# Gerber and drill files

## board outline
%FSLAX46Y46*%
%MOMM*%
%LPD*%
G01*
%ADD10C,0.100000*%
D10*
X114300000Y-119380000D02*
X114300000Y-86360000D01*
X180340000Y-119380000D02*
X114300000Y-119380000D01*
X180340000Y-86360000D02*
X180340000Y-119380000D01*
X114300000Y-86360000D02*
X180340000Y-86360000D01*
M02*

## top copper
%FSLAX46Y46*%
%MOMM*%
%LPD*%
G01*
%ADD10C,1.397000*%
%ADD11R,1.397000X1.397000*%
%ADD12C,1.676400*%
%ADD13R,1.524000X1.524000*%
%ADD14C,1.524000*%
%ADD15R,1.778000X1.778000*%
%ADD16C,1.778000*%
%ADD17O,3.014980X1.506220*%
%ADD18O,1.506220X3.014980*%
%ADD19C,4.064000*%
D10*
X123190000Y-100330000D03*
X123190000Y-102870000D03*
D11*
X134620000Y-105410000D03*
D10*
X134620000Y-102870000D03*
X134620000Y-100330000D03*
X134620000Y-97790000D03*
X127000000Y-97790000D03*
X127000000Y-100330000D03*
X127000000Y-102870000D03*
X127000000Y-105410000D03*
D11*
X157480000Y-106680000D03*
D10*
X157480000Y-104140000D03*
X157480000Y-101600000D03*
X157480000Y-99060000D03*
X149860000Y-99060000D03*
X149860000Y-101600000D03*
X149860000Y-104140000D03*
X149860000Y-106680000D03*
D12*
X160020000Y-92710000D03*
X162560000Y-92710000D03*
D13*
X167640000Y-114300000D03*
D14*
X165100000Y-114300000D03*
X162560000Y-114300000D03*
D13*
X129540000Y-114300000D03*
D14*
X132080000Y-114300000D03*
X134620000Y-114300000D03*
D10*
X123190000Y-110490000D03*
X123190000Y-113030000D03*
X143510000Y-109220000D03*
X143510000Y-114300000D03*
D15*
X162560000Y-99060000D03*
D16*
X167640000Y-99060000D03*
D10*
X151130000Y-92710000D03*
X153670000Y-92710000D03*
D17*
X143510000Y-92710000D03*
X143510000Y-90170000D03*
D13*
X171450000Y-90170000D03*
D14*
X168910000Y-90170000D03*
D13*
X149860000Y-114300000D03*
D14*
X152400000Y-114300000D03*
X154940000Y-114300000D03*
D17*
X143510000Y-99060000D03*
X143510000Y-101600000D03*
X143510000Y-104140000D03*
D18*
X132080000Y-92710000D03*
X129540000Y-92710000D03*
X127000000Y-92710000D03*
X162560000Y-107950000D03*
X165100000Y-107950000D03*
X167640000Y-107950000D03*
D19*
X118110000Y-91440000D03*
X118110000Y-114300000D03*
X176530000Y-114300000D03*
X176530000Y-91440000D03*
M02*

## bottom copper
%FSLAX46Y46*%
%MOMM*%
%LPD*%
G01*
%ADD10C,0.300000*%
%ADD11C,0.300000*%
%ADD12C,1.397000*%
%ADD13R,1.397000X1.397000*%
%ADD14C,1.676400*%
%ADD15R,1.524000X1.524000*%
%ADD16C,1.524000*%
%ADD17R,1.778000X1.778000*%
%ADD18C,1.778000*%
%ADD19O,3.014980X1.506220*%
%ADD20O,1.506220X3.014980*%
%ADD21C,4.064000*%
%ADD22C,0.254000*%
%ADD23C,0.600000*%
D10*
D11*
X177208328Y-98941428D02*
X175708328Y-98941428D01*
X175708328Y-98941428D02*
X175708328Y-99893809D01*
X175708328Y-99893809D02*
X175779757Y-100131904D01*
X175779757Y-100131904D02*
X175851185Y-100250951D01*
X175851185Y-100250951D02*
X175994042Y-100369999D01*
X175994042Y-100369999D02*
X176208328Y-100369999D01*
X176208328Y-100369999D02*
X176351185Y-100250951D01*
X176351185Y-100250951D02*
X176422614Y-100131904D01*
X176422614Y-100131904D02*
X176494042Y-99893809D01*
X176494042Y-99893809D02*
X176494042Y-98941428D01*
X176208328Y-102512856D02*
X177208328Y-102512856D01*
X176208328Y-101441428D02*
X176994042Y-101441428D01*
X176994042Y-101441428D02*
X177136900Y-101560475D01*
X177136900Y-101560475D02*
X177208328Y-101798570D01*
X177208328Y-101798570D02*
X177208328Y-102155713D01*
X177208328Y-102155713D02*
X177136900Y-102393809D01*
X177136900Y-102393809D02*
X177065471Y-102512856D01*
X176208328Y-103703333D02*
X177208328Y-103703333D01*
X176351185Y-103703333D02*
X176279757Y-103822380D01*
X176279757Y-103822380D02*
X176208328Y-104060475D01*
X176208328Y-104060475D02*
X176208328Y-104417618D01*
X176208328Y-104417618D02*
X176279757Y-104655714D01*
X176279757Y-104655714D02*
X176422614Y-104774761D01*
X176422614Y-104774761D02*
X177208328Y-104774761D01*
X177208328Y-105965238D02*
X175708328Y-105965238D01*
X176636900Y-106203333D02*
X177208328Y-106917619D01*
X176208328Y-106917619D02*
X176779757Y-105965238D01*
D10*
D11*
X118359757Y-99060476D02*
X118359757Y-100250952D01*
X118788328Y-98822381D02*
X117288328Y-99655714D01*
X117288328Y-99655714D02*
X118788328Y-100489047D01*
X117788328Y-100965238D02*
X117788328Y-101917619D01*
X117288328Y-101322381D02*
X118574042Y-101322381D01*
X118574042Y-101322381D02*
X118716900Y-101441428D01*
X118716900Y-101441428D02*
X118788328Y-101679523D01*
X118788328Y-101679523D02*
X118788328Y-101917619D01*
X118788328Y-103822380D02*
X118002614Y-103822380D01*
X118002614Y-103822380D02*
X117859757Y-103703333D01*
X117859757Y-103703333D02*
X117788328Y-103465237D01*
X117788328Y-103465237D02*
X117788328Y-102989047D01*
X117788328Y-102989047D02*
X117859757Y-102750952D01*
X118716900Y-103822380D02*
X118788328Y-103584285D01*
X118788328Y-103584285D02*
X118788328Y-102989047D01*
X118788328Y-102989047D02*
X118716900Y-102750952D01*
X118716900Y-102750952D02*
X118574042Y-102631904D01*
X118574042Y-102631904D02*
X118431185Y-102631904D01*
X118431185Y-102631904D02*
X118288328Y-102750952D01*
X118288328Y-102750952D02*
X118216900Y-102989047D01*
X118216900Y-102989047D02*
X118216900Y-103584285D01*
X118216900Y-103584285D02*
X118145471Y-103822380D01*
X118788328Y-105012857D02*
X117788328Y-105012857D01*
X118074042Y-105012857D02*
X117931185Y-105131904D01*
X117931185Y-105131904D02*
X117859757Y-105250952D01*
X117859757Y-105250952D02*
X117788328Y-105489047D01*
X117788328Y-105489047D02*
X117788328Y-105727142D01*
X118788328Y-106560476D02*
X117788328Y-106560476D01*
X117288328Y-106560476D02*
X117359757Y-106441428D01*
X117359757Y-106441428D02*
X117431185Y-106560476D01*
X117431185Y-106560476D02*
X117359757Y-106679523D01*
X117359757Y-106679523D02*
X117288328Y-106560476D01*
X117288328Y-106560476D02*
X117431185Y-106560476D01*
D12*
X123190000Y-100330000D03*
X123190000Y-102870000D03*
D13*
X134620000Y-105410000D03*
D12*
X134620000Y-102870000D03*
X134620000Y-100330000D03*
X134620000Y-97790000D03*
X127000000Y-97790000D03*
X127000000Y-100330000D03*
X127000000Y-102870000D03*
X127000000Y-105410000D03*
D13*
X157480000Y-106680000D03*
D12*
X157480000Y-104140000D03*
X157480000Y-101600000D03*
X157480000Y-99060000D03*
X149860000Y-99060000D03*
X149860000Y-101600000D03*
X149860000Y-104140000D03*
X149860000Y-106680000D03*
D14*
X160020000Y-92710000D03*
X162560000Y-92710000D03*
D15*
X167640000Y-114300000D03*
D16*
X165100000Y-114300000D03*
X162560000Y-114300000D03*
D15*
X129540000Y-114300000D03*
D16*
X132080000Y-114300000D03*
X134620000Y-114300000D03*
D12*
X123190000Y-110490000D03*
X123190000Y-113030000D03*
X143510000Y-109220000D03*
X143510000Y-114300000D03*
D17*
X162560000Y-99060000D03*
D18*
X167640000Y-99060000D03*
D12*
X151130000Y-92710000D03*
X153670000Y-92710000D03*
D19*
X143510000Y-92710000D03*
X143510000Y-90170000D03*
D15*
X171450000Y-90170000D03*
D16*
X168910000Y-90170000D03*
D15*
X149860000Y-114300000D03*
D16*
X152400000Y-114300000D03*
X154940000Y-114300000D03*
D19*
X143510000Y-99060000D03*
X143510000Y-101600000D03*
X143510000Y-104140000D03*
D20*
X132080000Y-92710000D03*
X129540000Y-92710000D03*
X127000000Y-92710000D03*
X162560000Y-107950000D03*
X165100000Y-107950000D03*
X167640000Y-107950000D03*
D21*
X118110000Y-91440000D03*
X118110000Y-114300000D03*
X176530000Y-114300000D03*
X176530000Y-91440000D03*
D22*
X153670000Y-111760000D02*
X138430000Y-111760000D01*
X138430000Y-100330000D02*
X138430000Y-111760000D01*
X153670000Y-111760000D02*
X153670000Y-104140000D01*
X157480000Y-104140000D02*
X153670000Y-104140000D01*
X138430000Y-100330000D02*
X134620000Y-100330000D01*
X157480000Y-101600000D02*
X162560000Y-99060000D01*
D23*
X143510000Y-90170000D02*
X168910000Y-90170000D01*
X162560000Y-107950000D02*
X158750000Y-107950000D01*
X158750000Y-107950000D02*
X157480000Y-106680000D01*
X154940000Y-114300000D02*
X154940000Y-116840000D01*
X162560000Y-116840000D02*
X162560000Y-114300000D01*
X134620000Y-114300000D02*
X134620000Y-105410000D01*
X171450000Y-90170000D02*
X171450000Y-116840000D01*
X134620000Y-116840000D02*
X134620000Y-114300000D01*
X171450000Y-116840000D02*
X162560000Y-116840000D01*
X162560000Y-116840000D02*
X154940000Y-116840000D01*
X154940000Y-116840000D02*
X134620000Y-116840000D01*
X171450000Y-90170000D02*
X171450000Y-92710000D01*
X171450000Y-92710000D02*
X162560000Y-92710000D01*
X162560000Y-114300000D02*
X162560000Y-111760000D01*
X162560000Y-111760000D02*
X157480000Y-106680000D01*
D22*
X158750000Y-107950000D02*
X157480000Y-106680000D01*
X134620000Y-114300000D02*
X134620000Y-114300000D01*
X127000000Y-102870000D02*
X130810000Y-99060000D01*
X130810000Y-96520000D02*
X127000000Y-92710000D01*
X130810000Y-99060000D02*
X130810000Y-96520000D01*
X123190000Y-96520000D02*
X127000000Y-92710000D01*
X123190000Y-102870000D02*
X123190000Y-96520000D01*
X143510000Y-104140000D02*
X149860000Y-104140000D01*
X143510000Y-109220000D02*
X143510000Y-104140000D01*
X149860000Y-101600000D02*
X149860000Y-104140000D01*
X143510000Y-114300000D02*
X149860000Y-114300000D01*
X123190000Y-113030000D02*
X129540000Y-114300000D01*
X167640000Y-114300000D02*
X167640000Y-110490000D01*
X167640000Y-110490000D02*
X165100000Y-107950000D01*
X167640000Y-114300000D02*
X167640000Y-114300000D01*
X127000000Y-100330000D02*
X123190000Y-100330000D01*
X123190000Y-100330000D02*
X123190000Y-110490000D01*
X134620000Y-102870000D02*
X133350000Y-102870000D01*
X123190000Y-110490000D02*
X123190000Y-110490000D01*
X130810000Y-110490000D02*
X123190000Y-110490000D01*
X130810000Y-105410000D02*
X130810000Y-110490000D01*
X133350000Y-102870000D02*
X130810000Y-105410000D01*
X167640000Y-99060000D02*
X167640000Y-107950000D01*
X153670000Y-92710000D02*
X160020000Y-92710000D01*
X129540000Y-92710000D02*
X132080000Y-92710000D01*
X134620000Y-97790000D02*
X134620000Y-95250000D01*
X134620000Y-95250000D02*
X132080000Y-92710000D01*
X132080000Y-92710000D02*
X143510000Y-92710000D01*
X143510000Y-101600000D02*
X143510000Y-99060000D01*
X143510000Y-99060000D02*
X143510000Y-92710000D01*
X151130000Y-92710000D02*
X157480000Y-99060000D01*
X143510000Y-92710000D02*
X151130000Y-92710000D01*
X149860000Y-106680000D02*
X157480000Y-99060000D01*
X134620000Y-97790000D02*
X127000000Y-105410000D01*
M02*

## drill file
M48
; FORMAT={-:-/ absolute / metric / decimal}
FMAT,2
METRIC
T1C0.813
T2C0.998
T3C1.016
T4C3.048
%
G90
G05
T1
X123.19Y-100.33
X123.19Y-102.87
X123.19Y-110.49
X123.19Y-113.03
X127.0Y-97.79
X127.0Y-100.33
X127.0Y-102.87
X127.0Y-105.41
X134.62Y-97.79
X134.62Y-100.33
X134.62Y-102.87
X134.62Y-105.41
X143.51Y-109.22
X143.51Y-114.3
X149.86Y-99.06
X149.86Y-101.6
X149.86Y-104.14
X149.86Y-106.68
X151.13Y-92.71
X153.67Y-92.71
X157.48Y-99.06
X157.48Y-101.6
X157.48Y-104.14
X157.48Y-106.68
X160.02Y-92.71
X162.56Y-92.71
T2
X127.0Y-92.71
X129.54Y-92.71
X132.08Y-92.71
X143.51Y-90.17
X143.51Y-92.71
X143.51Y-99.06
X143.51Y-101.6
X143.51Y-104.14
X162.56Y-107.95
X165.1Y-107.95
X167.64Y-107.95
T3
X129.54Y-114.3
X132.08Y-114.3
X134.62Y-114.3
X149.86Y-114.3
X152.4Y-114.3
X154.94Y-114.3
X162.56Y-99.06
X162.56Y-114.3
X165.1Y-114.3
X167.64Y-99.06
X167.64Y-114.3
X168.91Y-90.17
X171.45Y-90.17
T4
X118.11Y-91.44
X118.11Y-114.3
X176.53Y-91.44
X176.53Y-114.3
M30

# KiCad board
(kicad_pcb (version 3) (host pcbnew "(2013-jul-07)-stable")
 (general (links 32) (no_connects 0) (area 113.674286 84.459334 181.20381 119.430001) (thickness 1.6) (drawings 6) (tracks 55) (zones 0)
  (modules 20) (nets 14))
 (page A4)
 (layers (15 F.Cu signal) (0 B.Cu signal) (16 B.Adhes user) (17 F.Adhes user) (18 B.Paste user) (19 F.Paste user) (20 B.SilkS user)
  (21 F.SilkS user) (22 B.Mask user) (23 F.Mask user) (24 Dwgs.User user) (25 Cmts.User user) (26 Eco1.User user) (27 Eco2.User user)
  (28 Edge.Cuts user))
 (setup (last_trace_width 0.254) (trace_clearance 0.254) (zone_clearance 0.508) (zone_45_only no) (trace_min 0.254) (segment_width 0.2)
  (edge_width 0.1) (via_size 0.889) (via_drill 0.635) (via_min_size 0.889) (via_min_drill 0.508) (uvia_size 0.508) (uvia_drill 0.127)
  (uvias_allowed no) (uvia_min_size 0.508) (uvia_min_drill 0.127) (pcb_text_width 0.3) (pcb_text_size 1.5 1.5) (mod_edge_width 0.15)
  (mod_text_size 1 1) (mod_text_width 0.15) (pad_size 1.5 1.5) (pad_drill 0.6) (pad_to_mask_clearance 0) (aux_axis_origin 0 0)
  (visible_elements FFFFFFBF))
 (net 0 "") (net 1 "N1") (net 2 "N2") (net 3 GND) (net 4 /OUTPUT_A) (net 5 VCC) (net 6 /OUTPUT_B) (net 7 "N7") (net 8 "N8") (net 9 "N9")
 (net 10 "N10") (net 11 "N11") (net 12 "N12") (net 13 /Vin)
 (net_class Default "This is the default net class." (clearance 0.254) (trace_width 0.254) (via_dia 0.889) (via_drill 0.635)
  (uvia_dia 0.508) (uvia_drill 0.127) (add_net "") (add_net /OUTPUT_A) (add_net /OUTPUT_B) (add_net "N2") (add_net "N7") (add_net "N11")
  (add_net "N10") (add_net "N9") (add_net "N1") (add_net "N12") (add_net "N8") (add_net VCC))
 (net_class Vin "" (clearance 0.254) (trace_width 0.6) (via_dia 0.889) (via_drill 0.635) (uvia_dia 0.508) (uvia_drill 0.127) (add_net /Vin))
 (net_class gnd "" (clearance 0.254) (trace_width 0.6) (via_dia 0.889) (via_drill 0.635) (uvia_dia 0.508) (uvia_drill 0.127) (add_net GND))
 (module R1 (layer F.Cu) (at 123.19 101.6 270) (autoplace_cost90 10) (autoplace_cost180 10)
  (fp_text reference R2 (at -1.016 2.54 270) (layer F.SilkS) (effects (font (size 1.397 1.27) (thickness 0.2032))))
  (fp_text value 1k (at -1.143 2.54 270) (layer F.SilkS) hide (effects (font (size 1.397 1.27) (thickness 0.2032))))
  (pad 1 thru_hole circle (at -1.27 0 270) (size 1.397 1.397) (drill 0.8128) (layers *.Cu *.Mask F.SilkS) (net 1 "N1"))
  (pad 2 thru_hole circle (at 1.27 0 270) (size 1.397 1.397) (drill 0.8128) (layers *.Cu *.Mask F.SilkS) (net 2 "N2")))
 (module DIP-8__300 (layer F.Cu) (at 130.81 101.6 90)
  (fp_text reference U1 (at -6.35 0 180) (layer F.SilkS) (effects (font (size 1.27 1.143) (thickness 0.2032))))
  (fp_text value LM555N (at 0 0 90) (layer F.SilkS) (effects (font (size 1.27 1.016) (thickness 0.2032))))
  (pad 1 thru_hole rect (at -3.81 3.81 90) (size 1.397 1.397) (drill 0.8128) (layers *.Cu *.Mask F.SilkS) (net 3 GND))
  (pad 2 thru_hole circle (at -1.27 3.81 90) (size 1.397 1.397) (drill 0.8128) (layers *.Cu *.Mask F.SilkS) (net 1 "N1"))
  (pad 3 thru_hole circle (at 1.27 3.81 90) (size 1.397 1.397) (drill 0.8128) (layers *.Cu *.Mask F.SilkS) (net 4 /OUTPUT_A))
  (pad 4 thru_hole circle (at 3.81 3.81 90) (size 1.397 1.397) (drill 0.8128) (layers *.Cu *.Mask F.SilkS) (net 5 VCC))
  (pad 5 thru_hole circle (at 3.81 -3.81 90) (size 1.397 1.397) (drill 0.8128) (layers *.Cu *.Mask F.SilkS))
  (pad 6 thru_hole circle (at 1.27 -3.81 90) (size 1.397 1.397) (drill 0.8128) (layers *.Cu *.Mask F.SilkS) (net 1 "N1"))
  (pad 7 thru_hole circle (at -1.27 -3.81 90) (size 1.397 1.397) (drill 0.8128) (layers *.Cu *.Mask F.SilkS) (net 2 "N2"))
  (pad 8 thru_hole circle (at -3.81 -3.81 90) (size 1.397 1.397) (drill 0.8128) (layers *.Cu *.Mask F.SilkS) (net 5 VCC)))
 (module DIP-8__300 (layer F.Cu) (at 153.67 102.87 90)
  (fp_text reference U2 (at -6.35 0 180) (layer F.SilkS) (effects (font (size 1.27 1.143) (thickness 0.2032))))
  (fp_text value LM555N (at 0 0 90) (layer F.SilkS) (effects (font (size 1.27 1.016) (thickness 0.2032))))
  (pad 1 thru_hole rect (at -3.81 3.81 90) (size 1.397 1.397) (drill 0.8128) (layers *.Cu *.Mask F.SilkS) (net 3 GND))
  (pad 2 thru_hole circle (at -1.27 3.81 90) (size 1.397 1.397) (drill 0.8128) (layers *.Cu *.Mask F.SilkS) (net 4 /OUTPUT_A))
  (pad 3 thru_hole circle (at 1.27 3.81 90) (size 1.397 1.397) (drill 0.8128) (layers *.Cu *.Mask F.SilkS) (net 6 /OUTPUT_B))
  (pad 4 thru_hole circle (at 3.81 3.81 90) (size 1.397 1.397) (drill 0.8128) (layers *.Cu *.Mask F.SilkS) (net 5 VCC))
  (pad 5 thru_hole circle (at 3.81 -3.81 90) (size 1.397 1.397) (drill 0.8128) (layers *.Cu *.Mask F.SilkS))
  (pad 6 thru_hole circle (at 1.27 -3.81 90) (size 1.397 1.397) (drill 0.8128) (layers *.Cu *.Mask F.SilkS) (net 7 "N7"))
  (pad 7 thru_hole circle (at -1.27 -3.81 90) (size 1.397 1.397) (drill 0.8128) (layers *.Cu *.Mask F.SilkS) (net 7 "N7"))
  (pad 8 thru_hole circle (at -3.81 -3.81 90) (size 1.397 1.397) (drill 0.8128) (layers *.Cu *.Mask F.SilkS) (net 5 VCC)))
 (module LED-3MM (layer F.Cu) (at 161.29 92.71)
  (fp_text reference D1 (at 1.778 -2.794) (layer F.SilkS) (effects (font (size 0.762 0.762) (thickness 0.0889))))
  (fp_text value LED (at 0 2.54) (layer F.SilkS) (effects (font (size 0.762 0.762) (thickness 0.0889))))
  (pad 1 thru_hole circle (at -1.27 0) (size 1.6764 1.6764) (drill 0.8128) (layers *.Cu *.Mask F.SilkS) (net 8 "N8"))
  (pad 2 thru_hole circle (at 1.27 0) (size 1.6764 1.6764) (drill 0.8128) (layers *.Cu *.Mask F.SilkS) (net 3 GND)))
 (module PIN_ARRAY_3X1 (layer F.Cu) (at 165.1 114.3 180)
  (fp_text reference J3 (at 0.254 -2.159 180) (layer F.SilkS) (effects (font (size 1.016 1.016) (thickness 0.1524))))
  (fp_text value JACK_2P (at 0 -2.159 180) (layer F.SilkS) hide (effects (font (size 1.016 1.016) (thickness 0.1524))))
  (pad 1 thru_hole rect (at -2.54 0 180) (size 1.524 1.524) (drill 1.016) (layers *.Cu *.Mask F.SilkS) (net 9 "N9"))
  (pad 2 thru_hole circle (at 0 0 180) (size 1.524 1.524) (drill 1.016) (layers *.Cu *.Mask F.SilkS))
  (pad 3 thru_hole circle (at 2.54 0 180) (size 1.524 1.524) (drill 1.016) (layers *.Cu *.Mask F.SilkS) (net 3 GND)))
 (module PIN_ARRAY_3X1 (layer F.Cu) (at 132.08 114.3)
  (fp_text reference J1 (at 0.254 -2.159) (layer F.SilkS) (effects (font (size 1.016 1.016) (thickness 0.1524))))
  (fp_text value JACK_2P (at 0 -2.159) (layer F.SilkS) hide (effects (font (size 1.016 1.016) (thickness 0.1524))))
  (pad 1 thru_hole rect (at -2.54 0) (size 1.524 1.524) (drill 1.016) (layers *.Cu *.Mask F.SilkS) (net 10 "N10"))
  (pad 2 thru_hole circle (at 0 0) (size 1.524 1.524) (drill 1.016) (layers *.Cu *.Mask F.SilkS))
  (pad 3 thru_hole circle (at 2.54 0) (size 1.524 1.524) (drill 1.016) (layers *.Cu *.Mask F.SilkS) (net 3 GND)))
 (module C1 (layer F.Cu) (at 123.19 111.76 270)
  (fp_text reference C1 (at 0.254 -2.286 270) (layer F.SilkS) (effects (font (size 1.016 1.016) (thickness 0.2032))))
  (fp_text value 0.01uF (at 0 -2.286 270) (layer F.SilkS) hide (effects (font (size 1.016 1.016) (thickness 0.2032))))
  (pad 1 thru_hole circle (at -1.27 0 270) (size 1.397 1.397) (drill 0.8128) (layers *.Cu *.Mask F.SilkS) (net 1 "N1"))
  (pad 2 thru_hole circle (at 1.27 0 270) (size 1.397 1.397) (drill 0.8128) (layers *.Cu *.Mask F.SilkS) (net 10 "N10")))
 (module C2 (layer F.Cu) (at 143.51 111.76 270)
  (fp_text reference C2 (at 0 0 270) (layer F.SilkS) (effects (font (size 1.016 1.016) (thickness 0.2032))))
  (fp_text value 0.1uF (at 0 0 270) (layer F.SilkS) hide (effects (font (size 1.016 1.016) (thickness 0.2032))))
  (pad 1 thru_hole circle (at -2.54 0 270) (size 1.397 1.397) (drill 0.8128) (layers *.Cu *.Mask F.SilkS) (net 7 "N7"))
  (pad 2 thru_hole circle (at 2.54 0 270) (size 1.397 1.397) (drill 0.8128) (layers *.Cu *.Mask F.SilkS) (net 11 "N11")))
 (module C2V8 (layer F.Cu) (at 165.1 99.06)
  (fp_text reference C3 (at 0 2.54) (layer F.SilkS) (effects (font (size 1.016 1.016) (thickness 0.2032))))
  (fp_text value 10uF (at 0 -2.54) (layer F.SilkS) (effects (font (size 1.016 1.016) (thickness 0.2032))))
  (pad 1 thru_hole rect (at -2.54 0) (size 1.778 1.778) (drill 1.016) (layers *.Cu *.Mask F.SilkS) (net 6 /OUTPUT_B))
  (pad 2 thru_hole circle (at 2.54 0) (size 1.778 1.778) (drill 1.016) (layers *.Cu *.Mask F.SilkS) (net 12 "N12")))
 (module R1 (layer F.Cu) (at 152.4 92.71) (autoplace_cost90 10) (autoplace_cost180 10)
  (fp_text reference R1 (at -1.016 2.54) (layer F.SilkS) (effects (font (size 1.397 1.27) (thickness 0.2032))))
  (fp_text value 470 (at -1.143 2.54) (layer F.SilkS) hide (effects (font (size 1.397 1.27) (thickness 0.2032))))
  (pad 1 thru_hole circle (at -1.27 0) (size 1.397 1.397) (drill 0.8128) (layers *.Cu *.Mask F.SilkS) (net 5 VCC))
  (pad 2 thru_hole circle (at 1.27 0) (size 1.397 1.397) (drill 0.8128) (layers *.Cu *.Mask F.SilkS) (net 8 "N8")))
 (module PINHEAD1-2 (layer F.Cu) (at 143.51 91.44 90)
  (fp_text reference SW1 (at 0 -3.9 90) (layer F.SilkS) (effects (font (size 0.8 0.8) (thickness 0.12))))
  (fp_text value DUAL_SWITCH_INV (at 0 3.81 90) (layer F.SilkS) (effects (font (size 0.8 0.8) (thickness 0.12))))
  (pad 1 thru_hole oval (at -1.27 0 90) (size 1.50622 3.01498) (drill 0.99822) (layers *.Cu *.Mask F.SilkS) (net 5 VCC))
  (pad 2 thru_hole oval (at 1.27 0 90) (size 1.50622 3.01498) (drill 0.99822) (layers *.Cu *.Mask F.SilkS) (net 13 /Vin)))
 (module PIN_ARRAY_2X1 (layer F.Cu) (at 170.18 90.17 180)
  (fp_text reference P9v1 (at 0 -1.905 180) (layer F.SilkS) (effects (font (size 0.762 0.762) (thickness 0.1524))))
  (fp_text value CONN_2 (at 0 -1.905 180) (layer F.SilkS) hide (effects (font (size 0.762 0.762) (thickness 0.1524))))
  (pad 1 thru_hole rect (at -1.27 0 180) (size 1.524 1.524) (drill 1.016) (layers *.Cu *.Mask F.SilkS) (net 3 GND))
  (pad 2 thru_hole circle (at 1.27 0 180) (size 1.524 1.524) (drill 1.016) (layers *.Cu *.Mask F.SilkS) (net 13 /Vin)))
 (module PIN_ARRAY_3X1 (layer F.Cu) (at 152.4 114.3)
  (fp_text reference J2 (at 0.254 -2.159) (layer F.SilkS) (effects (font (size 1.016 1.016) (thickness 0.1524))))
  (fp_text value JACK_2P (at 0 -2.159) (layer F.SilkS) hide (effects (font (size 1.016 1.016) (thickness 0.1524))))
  (pad 1 thru_hole rect (at -2.54 0) (size 1.524 1.524) (drill 1.016) (layers *.Cu *.Mask F.SilkS) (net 11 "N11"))
  (pad 2 thru_hole circle (at 0 0) (size 1.524 1.524) (drill 1.016) (layers *.Cu *.Mask F.SilkS))
  (pad 3 thru_hole circle (at 2.54 0) (size 1.524 1.524) (drill 1.016) (layers *.Cu *.Mask F.SilkS) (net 3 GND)))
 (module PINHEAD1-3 (layer F.Cu) (at 143.51 101.6 270)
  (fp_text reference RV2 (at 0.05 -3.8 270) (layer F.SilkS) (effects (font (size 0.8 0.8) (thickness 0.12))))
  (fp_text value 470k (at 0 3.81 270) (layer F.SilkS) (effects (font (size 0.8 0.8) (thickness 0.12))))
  (pad 1 thru_hole oval (at -2.54 0 270) (size 1.50622 3.01498) (drill 0.99822) (layers *.Cu *.Mask F.SilkS) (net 5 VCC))
  (pad 2 thru_hole oval (at 0 0 270) (size 1.50622 3.01498) (drill 0.99822) (layers *.Cu *.Mask F.SilkS) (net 5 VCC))
  (pad 3 thru_hole oval (at 2.54 0 270) (size 1.50622 3.01498) (drill 0.99822) (layers *.Cu *.Mask F.SilkS) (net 7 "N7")))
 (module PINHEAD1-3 (layer F.Cu) (at 129.54 92.71 180)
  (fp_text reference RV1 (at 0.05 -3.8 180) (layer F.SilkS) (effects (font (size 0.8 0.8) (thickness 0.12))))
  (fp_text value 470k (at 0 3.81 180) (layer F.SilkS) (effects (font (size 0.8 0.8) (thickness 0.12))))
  (pad 1 thru_hole oval (at -2.54 0 180) (size 1.50622 3.01498) (drill 0.99822) (layers *.Cu *.Mask F.SilkS) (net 5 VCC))
  (pad 2 thru_hole oval (at 0 0 180) (size 1.50622 3.01498) (drill 0.99822) (layers *.Cu *.Mask F.SilkS) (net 5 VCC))
  (pad 3 thru_hole oval (at 2.54 0 180) (size 1.50622 3.01498) (drill 0.99822) (layers *.Cu *.Mask F.SilkS) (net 2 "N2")))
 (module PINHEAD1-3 (layer F.Cu) (at 165.1 107.95)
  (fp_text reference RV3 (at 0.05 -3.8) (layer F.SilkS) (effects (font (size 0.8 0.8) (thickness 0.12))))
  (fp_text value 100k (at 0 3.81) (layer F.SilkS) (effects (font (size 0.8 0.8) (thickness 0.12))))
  (pad 1 thru_hole oval (at -2.54 0) (size 1.50622 3.01498) (drill 0.99822) (layers *.Cu *.Mask F.SilkS) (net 3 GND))
  (pad 2 thru_hole oval (at 0 0) (size 1.50622 3.01498) (drill 0.99822) (layers *.Cu *.Mask F.SilkS) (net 9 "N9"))
  (pad 3 thru_hole oval (at 2.54 0) (size 1.50622 3.01498) (drill 0.99822) (layers *.Cu *.Mask F.SilkS) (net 12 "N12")))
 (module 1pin (layer F.Cu) (at 118.11 91.44)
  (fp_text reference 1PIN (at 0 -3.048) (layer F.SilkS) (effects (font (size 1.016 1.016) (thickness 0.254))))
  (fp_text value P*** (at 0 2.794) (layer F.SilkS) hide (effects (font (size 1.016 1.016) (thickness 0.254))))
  (pad 1 thru_hole circle (at 0 0) (size 4.064 4.064) (drill 3.048) (layers *.Cu *.Mask F.SilkS)))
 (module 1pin (layer F.Cu) (at 118.11 114.3)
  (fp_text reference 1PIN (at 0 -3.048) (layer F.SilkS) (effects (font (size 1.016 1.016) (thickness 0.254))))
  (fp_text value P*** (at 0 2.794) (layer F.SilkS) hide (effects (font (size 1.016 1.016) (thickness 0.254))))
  (pad 1 thru_hole circle (at 0 0) (size 4.064 4.064) (drill 3.048) (layers *.Cu *.Mask F.SilkS)))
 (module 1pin (layer F.Cu) (at 176.53 114.3)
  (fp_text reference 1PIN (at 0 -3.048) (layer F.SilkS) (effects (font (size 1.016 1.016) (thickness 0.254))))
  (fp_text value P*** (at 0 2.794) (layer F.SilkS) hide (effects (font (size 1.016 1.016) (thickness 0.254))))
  (pad 1 thru_hole circle (at 0 0) (size 4.064 4.064) (drill 3.048) (layers *.Cu *.Mask F.SilkS)))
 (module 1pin (layer F.Cu) (at 176.53 91.44)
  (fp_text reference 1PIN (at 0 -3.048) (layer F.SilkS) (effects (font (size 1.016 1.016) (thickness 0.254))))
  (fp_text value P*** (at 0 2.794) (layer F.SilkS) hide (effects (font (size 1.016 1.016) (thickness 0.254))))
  (pad 1 thru_hole circle (at 0 0) (size 4.064 4.064) (drill 3.048) (layers *.Cu *.Mask F.SilkS)))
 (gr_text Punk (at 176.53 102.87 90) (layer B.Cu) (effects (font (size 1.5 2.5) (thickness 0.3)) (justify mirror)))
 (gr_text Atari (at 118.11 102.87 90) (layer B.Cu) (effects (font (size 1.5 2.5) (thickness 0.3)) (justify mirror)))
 (gr_line (start 114.3 119.38) (end 114.3 86.36) (angle 90) (layer Edge.Cuts) (width 0.1))
 (gr_line (start 180.34 119.38) (end 114.3 119.38) (angle 90) (layer Edge.Cuts) (width 0.1))
 (gr_line (start 180.34 86.36) (end 180.34 119.38) (angle 90) (layer Edge.Cuts) (width 0.1))
 (gr_line (start 114.3 86.36) (end 180.34 86.36) (angle 90) (layer Edge.Cuts) (width 0.1))
 (segment (start 153.67 111.76) (end 138.43 111.76) (width 0.254) (layer B.Cu) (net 4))
 (segment (start 138.43 100.33) (end 138.43 111.76) (width 0.254) (layer B.Cu) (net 4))
 (segment (start 153.67 111.76) (end 153.67 104.14) (width 0.254) (layer B.Cu) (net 4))
 (segment (start 157.48 104.14) (end 153.67 104.14) (width 0.254) (layer B.Cu) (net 4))
 (segment (start 138.43 100.33) (end 134.62 100.33) (width 0.254) (layer B.Cu) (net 4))
 (segment (start 157.48 101.6) (end 162.56 99.06) (width 0.254) (layer B.Cu) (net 6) (status 20))
 (segment (start 143.51 90.17) (end 168.91 90.17) (width 0.6) (layer B.Cu) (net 13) (status C00000))
 (segment (start 162.56 107.95) (end 158.75 107.95) (width 0.6) (layer B.Cu) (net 3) (status 400000))
 (segment (start 158.75 107.95) (end 157.48 106.68) (width 0.6) (layer B.Cu) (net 3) (status 800000))
 (segment (start 154.94 114.3) (end 154.94 116.84) (width 0.6) (layer B.Cu) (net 3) (status 400000))
 (segment (start 162.56 116.84) (end 162.56 114.3) (width 0.6) (layer B.Cu) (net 3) (status 800000))
 (segment (start 134.62 114.3) (end 134.62 105.41) (width 0.6) (layer B.Cu) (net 3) (status C00000))
 (segment (start 171.45 90.17) (end 171.45 116.84) (width 0.6) (layer B.Cu) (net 3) (status 400000))
 (segment (start 134.62 116.84) (end 134.62 114.3) (width 0.6) (layer B.Cu) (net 3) (status 800000))
 (segment (start 171.45 116.84) (end 162.56 116.84) (width 0.6) (layer B.Cu) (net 3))
 (segment (start 162.56 116.84) (end 154.94 116.84) (width 0.6) (layer B.Cu) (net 3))
 (segment (start 154.94 116.84) (end 134.62 116.84) (width 0.6) (layer B.Cu) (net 3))
 (segment (start 171.45 90.17) (end 171.45 92.71) (width 0.6) (layer B.Cu) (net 3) (status 400000))
 (segment (start 171.45 92.71) (end 162.56 92.71) (width 0.6) (layer B.Cu) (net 3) (status 800000))
 (segment (start 162.56 114.3) (end 162.56 111.76) (width 0.6) (layer B.Cu) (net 3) (status 400000))
 (segment (start 162.56 111.76) (end 157.48 106.68) (width 0.6) (layer B.Cu) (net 3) (status 800000))
 (segment (start 158.75 107.95) (end 157.48 106.68) (width 0.254) (layer B.Cu) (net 3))
 (segment (start 134.62 114.3) (end 134.62 114.3) (width 0.254) (layer B.Cu) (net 3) (status 30))
 (segment (start 127 102.87) (end 130.81 99.06) (width 0.254) (layer B.Cu) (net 2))
 (segment (start 130.81 96.52) (end 127 92.71) (width 0.254) (layer B.Cu) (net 2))
 (segment (start 130.81 99.06) (end 130.81 96.52) (width 0.254) (layer B.Cu) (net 2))
 (segment (start 123.19 96.52) (end 127 92.71) (width 0.254) (layer B.Cu) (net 2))
 (segment (start 123.19 102.87) (end 123.19 96.52) (width 0.254) (layer B.Cu) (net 2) (status 10))
 (segment (start 143.51 104.14) (end 149.86 104.14) (width 0.254) (layer B.Cu) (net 7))
 (segment (start 143.51 109.22) (end 143.51 104.14) (width 0.254) (layer B.Cu) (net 7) (status 10))
 (segment (start 149.86 101.6) (end 149.86 104.14) (width 0.254) (layer B.Cu) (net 7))
 (segment (start 143.51 114.3) (end 149.86 114.3) (width 0.254) (layer B.Cu) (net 11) (status 20))
 (segment (start 123.19 113.03) (end 129.54 114.3) (width 0.254) (layer B.Cu) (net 10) (status 20))
 (segment (start 167.64 114.3) (end 167.64 110.49) (width 0.254) (layer B.Cu) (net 9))
 (segment (start 167.64 110.49) (end 165.1 107.95) (width 0.254) (layer B.Cu) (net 9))
 (segment (start 167.64 114.3) (end 167.64 114.3) (width 0.254) (layer B.Cu) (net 9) (status 30))
 (segment (start 127 100.33) (end 123.19 100.33) (width 0.254) (layer B.Cu) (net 1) (status 20))
 (segment (start 123.19 100.33) (end 123.19 110.49) (width 0.254) (layer B.Cu) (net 1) (status 10))
 (segment (start 134.62 102.87) (end 133.35 102.87) (width 0.254) (layer B.Cu) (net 1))
 (segment (start 123.19 110.49) (end 123.19 110.49) (width 0.254) (layer B.Cu) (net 1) (status 30))
 (segment (start 130.81 110.49) (end 123.19 110.49) (width 0.254) (layer B.Cu) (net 1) (status 20))
 (segment (start 130.81 105.41) (end 130.81 110.49) (width 0.254) (layer B.Cu) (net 1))
 (segment (start 133.35 102.87) (end 130.81 105.41) (width 0.254) (layer B.Cu) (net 1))
 (segment (start 167.64 99.06) (end 167.64 107.95) (width 0.254) (layer B.Cu) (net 12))
 (segment (start 153.67 92.71) (end 160.02 92.71) (width 0.254) (layer B.Cu) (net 8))
 (segment (start 129.54 92.71) (end 132.08 92.71) (width 0.254) (layer B.Cu) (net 5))
 (segment (start 134.62 97.79) (end 134.62 95.25) (width 0.254) (layer B.Cu) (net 5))
 (segment (start 134.62 95.25) (end 132.08 92.71) (width 0.254) (layer B.Cu) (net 5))
 (segment (start 132.08 92.71) (end 143.51 92.71) (width 0.254) (layer B.Cu) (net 5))
 (segment (start 143.51 101.6) (end 143.51 99.06) (width 0.254) (layer B.Cu) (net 5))
 (segment (start 143.51 99.06) (end 143.51 92.71) (width 0.254) (layer B.Cu) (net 5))
 (segment (start 151.13 92.71) (end 157.48 99.06) (width 0.254) (layer B.Cu) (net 5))
 (segment (start 143.51 92.71) (end 151.13 92.71) (width 0.254) (layer B.Cu) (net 5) (status 10))
 (segment (start 149.86 106.68) (end 157.48 99.06) (width 0.254) (layer B.Cu) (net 5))
 (segment (start 134.62 97.79) (end 127 105.41) (width 0.254) (layer B.Cu) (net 5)))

